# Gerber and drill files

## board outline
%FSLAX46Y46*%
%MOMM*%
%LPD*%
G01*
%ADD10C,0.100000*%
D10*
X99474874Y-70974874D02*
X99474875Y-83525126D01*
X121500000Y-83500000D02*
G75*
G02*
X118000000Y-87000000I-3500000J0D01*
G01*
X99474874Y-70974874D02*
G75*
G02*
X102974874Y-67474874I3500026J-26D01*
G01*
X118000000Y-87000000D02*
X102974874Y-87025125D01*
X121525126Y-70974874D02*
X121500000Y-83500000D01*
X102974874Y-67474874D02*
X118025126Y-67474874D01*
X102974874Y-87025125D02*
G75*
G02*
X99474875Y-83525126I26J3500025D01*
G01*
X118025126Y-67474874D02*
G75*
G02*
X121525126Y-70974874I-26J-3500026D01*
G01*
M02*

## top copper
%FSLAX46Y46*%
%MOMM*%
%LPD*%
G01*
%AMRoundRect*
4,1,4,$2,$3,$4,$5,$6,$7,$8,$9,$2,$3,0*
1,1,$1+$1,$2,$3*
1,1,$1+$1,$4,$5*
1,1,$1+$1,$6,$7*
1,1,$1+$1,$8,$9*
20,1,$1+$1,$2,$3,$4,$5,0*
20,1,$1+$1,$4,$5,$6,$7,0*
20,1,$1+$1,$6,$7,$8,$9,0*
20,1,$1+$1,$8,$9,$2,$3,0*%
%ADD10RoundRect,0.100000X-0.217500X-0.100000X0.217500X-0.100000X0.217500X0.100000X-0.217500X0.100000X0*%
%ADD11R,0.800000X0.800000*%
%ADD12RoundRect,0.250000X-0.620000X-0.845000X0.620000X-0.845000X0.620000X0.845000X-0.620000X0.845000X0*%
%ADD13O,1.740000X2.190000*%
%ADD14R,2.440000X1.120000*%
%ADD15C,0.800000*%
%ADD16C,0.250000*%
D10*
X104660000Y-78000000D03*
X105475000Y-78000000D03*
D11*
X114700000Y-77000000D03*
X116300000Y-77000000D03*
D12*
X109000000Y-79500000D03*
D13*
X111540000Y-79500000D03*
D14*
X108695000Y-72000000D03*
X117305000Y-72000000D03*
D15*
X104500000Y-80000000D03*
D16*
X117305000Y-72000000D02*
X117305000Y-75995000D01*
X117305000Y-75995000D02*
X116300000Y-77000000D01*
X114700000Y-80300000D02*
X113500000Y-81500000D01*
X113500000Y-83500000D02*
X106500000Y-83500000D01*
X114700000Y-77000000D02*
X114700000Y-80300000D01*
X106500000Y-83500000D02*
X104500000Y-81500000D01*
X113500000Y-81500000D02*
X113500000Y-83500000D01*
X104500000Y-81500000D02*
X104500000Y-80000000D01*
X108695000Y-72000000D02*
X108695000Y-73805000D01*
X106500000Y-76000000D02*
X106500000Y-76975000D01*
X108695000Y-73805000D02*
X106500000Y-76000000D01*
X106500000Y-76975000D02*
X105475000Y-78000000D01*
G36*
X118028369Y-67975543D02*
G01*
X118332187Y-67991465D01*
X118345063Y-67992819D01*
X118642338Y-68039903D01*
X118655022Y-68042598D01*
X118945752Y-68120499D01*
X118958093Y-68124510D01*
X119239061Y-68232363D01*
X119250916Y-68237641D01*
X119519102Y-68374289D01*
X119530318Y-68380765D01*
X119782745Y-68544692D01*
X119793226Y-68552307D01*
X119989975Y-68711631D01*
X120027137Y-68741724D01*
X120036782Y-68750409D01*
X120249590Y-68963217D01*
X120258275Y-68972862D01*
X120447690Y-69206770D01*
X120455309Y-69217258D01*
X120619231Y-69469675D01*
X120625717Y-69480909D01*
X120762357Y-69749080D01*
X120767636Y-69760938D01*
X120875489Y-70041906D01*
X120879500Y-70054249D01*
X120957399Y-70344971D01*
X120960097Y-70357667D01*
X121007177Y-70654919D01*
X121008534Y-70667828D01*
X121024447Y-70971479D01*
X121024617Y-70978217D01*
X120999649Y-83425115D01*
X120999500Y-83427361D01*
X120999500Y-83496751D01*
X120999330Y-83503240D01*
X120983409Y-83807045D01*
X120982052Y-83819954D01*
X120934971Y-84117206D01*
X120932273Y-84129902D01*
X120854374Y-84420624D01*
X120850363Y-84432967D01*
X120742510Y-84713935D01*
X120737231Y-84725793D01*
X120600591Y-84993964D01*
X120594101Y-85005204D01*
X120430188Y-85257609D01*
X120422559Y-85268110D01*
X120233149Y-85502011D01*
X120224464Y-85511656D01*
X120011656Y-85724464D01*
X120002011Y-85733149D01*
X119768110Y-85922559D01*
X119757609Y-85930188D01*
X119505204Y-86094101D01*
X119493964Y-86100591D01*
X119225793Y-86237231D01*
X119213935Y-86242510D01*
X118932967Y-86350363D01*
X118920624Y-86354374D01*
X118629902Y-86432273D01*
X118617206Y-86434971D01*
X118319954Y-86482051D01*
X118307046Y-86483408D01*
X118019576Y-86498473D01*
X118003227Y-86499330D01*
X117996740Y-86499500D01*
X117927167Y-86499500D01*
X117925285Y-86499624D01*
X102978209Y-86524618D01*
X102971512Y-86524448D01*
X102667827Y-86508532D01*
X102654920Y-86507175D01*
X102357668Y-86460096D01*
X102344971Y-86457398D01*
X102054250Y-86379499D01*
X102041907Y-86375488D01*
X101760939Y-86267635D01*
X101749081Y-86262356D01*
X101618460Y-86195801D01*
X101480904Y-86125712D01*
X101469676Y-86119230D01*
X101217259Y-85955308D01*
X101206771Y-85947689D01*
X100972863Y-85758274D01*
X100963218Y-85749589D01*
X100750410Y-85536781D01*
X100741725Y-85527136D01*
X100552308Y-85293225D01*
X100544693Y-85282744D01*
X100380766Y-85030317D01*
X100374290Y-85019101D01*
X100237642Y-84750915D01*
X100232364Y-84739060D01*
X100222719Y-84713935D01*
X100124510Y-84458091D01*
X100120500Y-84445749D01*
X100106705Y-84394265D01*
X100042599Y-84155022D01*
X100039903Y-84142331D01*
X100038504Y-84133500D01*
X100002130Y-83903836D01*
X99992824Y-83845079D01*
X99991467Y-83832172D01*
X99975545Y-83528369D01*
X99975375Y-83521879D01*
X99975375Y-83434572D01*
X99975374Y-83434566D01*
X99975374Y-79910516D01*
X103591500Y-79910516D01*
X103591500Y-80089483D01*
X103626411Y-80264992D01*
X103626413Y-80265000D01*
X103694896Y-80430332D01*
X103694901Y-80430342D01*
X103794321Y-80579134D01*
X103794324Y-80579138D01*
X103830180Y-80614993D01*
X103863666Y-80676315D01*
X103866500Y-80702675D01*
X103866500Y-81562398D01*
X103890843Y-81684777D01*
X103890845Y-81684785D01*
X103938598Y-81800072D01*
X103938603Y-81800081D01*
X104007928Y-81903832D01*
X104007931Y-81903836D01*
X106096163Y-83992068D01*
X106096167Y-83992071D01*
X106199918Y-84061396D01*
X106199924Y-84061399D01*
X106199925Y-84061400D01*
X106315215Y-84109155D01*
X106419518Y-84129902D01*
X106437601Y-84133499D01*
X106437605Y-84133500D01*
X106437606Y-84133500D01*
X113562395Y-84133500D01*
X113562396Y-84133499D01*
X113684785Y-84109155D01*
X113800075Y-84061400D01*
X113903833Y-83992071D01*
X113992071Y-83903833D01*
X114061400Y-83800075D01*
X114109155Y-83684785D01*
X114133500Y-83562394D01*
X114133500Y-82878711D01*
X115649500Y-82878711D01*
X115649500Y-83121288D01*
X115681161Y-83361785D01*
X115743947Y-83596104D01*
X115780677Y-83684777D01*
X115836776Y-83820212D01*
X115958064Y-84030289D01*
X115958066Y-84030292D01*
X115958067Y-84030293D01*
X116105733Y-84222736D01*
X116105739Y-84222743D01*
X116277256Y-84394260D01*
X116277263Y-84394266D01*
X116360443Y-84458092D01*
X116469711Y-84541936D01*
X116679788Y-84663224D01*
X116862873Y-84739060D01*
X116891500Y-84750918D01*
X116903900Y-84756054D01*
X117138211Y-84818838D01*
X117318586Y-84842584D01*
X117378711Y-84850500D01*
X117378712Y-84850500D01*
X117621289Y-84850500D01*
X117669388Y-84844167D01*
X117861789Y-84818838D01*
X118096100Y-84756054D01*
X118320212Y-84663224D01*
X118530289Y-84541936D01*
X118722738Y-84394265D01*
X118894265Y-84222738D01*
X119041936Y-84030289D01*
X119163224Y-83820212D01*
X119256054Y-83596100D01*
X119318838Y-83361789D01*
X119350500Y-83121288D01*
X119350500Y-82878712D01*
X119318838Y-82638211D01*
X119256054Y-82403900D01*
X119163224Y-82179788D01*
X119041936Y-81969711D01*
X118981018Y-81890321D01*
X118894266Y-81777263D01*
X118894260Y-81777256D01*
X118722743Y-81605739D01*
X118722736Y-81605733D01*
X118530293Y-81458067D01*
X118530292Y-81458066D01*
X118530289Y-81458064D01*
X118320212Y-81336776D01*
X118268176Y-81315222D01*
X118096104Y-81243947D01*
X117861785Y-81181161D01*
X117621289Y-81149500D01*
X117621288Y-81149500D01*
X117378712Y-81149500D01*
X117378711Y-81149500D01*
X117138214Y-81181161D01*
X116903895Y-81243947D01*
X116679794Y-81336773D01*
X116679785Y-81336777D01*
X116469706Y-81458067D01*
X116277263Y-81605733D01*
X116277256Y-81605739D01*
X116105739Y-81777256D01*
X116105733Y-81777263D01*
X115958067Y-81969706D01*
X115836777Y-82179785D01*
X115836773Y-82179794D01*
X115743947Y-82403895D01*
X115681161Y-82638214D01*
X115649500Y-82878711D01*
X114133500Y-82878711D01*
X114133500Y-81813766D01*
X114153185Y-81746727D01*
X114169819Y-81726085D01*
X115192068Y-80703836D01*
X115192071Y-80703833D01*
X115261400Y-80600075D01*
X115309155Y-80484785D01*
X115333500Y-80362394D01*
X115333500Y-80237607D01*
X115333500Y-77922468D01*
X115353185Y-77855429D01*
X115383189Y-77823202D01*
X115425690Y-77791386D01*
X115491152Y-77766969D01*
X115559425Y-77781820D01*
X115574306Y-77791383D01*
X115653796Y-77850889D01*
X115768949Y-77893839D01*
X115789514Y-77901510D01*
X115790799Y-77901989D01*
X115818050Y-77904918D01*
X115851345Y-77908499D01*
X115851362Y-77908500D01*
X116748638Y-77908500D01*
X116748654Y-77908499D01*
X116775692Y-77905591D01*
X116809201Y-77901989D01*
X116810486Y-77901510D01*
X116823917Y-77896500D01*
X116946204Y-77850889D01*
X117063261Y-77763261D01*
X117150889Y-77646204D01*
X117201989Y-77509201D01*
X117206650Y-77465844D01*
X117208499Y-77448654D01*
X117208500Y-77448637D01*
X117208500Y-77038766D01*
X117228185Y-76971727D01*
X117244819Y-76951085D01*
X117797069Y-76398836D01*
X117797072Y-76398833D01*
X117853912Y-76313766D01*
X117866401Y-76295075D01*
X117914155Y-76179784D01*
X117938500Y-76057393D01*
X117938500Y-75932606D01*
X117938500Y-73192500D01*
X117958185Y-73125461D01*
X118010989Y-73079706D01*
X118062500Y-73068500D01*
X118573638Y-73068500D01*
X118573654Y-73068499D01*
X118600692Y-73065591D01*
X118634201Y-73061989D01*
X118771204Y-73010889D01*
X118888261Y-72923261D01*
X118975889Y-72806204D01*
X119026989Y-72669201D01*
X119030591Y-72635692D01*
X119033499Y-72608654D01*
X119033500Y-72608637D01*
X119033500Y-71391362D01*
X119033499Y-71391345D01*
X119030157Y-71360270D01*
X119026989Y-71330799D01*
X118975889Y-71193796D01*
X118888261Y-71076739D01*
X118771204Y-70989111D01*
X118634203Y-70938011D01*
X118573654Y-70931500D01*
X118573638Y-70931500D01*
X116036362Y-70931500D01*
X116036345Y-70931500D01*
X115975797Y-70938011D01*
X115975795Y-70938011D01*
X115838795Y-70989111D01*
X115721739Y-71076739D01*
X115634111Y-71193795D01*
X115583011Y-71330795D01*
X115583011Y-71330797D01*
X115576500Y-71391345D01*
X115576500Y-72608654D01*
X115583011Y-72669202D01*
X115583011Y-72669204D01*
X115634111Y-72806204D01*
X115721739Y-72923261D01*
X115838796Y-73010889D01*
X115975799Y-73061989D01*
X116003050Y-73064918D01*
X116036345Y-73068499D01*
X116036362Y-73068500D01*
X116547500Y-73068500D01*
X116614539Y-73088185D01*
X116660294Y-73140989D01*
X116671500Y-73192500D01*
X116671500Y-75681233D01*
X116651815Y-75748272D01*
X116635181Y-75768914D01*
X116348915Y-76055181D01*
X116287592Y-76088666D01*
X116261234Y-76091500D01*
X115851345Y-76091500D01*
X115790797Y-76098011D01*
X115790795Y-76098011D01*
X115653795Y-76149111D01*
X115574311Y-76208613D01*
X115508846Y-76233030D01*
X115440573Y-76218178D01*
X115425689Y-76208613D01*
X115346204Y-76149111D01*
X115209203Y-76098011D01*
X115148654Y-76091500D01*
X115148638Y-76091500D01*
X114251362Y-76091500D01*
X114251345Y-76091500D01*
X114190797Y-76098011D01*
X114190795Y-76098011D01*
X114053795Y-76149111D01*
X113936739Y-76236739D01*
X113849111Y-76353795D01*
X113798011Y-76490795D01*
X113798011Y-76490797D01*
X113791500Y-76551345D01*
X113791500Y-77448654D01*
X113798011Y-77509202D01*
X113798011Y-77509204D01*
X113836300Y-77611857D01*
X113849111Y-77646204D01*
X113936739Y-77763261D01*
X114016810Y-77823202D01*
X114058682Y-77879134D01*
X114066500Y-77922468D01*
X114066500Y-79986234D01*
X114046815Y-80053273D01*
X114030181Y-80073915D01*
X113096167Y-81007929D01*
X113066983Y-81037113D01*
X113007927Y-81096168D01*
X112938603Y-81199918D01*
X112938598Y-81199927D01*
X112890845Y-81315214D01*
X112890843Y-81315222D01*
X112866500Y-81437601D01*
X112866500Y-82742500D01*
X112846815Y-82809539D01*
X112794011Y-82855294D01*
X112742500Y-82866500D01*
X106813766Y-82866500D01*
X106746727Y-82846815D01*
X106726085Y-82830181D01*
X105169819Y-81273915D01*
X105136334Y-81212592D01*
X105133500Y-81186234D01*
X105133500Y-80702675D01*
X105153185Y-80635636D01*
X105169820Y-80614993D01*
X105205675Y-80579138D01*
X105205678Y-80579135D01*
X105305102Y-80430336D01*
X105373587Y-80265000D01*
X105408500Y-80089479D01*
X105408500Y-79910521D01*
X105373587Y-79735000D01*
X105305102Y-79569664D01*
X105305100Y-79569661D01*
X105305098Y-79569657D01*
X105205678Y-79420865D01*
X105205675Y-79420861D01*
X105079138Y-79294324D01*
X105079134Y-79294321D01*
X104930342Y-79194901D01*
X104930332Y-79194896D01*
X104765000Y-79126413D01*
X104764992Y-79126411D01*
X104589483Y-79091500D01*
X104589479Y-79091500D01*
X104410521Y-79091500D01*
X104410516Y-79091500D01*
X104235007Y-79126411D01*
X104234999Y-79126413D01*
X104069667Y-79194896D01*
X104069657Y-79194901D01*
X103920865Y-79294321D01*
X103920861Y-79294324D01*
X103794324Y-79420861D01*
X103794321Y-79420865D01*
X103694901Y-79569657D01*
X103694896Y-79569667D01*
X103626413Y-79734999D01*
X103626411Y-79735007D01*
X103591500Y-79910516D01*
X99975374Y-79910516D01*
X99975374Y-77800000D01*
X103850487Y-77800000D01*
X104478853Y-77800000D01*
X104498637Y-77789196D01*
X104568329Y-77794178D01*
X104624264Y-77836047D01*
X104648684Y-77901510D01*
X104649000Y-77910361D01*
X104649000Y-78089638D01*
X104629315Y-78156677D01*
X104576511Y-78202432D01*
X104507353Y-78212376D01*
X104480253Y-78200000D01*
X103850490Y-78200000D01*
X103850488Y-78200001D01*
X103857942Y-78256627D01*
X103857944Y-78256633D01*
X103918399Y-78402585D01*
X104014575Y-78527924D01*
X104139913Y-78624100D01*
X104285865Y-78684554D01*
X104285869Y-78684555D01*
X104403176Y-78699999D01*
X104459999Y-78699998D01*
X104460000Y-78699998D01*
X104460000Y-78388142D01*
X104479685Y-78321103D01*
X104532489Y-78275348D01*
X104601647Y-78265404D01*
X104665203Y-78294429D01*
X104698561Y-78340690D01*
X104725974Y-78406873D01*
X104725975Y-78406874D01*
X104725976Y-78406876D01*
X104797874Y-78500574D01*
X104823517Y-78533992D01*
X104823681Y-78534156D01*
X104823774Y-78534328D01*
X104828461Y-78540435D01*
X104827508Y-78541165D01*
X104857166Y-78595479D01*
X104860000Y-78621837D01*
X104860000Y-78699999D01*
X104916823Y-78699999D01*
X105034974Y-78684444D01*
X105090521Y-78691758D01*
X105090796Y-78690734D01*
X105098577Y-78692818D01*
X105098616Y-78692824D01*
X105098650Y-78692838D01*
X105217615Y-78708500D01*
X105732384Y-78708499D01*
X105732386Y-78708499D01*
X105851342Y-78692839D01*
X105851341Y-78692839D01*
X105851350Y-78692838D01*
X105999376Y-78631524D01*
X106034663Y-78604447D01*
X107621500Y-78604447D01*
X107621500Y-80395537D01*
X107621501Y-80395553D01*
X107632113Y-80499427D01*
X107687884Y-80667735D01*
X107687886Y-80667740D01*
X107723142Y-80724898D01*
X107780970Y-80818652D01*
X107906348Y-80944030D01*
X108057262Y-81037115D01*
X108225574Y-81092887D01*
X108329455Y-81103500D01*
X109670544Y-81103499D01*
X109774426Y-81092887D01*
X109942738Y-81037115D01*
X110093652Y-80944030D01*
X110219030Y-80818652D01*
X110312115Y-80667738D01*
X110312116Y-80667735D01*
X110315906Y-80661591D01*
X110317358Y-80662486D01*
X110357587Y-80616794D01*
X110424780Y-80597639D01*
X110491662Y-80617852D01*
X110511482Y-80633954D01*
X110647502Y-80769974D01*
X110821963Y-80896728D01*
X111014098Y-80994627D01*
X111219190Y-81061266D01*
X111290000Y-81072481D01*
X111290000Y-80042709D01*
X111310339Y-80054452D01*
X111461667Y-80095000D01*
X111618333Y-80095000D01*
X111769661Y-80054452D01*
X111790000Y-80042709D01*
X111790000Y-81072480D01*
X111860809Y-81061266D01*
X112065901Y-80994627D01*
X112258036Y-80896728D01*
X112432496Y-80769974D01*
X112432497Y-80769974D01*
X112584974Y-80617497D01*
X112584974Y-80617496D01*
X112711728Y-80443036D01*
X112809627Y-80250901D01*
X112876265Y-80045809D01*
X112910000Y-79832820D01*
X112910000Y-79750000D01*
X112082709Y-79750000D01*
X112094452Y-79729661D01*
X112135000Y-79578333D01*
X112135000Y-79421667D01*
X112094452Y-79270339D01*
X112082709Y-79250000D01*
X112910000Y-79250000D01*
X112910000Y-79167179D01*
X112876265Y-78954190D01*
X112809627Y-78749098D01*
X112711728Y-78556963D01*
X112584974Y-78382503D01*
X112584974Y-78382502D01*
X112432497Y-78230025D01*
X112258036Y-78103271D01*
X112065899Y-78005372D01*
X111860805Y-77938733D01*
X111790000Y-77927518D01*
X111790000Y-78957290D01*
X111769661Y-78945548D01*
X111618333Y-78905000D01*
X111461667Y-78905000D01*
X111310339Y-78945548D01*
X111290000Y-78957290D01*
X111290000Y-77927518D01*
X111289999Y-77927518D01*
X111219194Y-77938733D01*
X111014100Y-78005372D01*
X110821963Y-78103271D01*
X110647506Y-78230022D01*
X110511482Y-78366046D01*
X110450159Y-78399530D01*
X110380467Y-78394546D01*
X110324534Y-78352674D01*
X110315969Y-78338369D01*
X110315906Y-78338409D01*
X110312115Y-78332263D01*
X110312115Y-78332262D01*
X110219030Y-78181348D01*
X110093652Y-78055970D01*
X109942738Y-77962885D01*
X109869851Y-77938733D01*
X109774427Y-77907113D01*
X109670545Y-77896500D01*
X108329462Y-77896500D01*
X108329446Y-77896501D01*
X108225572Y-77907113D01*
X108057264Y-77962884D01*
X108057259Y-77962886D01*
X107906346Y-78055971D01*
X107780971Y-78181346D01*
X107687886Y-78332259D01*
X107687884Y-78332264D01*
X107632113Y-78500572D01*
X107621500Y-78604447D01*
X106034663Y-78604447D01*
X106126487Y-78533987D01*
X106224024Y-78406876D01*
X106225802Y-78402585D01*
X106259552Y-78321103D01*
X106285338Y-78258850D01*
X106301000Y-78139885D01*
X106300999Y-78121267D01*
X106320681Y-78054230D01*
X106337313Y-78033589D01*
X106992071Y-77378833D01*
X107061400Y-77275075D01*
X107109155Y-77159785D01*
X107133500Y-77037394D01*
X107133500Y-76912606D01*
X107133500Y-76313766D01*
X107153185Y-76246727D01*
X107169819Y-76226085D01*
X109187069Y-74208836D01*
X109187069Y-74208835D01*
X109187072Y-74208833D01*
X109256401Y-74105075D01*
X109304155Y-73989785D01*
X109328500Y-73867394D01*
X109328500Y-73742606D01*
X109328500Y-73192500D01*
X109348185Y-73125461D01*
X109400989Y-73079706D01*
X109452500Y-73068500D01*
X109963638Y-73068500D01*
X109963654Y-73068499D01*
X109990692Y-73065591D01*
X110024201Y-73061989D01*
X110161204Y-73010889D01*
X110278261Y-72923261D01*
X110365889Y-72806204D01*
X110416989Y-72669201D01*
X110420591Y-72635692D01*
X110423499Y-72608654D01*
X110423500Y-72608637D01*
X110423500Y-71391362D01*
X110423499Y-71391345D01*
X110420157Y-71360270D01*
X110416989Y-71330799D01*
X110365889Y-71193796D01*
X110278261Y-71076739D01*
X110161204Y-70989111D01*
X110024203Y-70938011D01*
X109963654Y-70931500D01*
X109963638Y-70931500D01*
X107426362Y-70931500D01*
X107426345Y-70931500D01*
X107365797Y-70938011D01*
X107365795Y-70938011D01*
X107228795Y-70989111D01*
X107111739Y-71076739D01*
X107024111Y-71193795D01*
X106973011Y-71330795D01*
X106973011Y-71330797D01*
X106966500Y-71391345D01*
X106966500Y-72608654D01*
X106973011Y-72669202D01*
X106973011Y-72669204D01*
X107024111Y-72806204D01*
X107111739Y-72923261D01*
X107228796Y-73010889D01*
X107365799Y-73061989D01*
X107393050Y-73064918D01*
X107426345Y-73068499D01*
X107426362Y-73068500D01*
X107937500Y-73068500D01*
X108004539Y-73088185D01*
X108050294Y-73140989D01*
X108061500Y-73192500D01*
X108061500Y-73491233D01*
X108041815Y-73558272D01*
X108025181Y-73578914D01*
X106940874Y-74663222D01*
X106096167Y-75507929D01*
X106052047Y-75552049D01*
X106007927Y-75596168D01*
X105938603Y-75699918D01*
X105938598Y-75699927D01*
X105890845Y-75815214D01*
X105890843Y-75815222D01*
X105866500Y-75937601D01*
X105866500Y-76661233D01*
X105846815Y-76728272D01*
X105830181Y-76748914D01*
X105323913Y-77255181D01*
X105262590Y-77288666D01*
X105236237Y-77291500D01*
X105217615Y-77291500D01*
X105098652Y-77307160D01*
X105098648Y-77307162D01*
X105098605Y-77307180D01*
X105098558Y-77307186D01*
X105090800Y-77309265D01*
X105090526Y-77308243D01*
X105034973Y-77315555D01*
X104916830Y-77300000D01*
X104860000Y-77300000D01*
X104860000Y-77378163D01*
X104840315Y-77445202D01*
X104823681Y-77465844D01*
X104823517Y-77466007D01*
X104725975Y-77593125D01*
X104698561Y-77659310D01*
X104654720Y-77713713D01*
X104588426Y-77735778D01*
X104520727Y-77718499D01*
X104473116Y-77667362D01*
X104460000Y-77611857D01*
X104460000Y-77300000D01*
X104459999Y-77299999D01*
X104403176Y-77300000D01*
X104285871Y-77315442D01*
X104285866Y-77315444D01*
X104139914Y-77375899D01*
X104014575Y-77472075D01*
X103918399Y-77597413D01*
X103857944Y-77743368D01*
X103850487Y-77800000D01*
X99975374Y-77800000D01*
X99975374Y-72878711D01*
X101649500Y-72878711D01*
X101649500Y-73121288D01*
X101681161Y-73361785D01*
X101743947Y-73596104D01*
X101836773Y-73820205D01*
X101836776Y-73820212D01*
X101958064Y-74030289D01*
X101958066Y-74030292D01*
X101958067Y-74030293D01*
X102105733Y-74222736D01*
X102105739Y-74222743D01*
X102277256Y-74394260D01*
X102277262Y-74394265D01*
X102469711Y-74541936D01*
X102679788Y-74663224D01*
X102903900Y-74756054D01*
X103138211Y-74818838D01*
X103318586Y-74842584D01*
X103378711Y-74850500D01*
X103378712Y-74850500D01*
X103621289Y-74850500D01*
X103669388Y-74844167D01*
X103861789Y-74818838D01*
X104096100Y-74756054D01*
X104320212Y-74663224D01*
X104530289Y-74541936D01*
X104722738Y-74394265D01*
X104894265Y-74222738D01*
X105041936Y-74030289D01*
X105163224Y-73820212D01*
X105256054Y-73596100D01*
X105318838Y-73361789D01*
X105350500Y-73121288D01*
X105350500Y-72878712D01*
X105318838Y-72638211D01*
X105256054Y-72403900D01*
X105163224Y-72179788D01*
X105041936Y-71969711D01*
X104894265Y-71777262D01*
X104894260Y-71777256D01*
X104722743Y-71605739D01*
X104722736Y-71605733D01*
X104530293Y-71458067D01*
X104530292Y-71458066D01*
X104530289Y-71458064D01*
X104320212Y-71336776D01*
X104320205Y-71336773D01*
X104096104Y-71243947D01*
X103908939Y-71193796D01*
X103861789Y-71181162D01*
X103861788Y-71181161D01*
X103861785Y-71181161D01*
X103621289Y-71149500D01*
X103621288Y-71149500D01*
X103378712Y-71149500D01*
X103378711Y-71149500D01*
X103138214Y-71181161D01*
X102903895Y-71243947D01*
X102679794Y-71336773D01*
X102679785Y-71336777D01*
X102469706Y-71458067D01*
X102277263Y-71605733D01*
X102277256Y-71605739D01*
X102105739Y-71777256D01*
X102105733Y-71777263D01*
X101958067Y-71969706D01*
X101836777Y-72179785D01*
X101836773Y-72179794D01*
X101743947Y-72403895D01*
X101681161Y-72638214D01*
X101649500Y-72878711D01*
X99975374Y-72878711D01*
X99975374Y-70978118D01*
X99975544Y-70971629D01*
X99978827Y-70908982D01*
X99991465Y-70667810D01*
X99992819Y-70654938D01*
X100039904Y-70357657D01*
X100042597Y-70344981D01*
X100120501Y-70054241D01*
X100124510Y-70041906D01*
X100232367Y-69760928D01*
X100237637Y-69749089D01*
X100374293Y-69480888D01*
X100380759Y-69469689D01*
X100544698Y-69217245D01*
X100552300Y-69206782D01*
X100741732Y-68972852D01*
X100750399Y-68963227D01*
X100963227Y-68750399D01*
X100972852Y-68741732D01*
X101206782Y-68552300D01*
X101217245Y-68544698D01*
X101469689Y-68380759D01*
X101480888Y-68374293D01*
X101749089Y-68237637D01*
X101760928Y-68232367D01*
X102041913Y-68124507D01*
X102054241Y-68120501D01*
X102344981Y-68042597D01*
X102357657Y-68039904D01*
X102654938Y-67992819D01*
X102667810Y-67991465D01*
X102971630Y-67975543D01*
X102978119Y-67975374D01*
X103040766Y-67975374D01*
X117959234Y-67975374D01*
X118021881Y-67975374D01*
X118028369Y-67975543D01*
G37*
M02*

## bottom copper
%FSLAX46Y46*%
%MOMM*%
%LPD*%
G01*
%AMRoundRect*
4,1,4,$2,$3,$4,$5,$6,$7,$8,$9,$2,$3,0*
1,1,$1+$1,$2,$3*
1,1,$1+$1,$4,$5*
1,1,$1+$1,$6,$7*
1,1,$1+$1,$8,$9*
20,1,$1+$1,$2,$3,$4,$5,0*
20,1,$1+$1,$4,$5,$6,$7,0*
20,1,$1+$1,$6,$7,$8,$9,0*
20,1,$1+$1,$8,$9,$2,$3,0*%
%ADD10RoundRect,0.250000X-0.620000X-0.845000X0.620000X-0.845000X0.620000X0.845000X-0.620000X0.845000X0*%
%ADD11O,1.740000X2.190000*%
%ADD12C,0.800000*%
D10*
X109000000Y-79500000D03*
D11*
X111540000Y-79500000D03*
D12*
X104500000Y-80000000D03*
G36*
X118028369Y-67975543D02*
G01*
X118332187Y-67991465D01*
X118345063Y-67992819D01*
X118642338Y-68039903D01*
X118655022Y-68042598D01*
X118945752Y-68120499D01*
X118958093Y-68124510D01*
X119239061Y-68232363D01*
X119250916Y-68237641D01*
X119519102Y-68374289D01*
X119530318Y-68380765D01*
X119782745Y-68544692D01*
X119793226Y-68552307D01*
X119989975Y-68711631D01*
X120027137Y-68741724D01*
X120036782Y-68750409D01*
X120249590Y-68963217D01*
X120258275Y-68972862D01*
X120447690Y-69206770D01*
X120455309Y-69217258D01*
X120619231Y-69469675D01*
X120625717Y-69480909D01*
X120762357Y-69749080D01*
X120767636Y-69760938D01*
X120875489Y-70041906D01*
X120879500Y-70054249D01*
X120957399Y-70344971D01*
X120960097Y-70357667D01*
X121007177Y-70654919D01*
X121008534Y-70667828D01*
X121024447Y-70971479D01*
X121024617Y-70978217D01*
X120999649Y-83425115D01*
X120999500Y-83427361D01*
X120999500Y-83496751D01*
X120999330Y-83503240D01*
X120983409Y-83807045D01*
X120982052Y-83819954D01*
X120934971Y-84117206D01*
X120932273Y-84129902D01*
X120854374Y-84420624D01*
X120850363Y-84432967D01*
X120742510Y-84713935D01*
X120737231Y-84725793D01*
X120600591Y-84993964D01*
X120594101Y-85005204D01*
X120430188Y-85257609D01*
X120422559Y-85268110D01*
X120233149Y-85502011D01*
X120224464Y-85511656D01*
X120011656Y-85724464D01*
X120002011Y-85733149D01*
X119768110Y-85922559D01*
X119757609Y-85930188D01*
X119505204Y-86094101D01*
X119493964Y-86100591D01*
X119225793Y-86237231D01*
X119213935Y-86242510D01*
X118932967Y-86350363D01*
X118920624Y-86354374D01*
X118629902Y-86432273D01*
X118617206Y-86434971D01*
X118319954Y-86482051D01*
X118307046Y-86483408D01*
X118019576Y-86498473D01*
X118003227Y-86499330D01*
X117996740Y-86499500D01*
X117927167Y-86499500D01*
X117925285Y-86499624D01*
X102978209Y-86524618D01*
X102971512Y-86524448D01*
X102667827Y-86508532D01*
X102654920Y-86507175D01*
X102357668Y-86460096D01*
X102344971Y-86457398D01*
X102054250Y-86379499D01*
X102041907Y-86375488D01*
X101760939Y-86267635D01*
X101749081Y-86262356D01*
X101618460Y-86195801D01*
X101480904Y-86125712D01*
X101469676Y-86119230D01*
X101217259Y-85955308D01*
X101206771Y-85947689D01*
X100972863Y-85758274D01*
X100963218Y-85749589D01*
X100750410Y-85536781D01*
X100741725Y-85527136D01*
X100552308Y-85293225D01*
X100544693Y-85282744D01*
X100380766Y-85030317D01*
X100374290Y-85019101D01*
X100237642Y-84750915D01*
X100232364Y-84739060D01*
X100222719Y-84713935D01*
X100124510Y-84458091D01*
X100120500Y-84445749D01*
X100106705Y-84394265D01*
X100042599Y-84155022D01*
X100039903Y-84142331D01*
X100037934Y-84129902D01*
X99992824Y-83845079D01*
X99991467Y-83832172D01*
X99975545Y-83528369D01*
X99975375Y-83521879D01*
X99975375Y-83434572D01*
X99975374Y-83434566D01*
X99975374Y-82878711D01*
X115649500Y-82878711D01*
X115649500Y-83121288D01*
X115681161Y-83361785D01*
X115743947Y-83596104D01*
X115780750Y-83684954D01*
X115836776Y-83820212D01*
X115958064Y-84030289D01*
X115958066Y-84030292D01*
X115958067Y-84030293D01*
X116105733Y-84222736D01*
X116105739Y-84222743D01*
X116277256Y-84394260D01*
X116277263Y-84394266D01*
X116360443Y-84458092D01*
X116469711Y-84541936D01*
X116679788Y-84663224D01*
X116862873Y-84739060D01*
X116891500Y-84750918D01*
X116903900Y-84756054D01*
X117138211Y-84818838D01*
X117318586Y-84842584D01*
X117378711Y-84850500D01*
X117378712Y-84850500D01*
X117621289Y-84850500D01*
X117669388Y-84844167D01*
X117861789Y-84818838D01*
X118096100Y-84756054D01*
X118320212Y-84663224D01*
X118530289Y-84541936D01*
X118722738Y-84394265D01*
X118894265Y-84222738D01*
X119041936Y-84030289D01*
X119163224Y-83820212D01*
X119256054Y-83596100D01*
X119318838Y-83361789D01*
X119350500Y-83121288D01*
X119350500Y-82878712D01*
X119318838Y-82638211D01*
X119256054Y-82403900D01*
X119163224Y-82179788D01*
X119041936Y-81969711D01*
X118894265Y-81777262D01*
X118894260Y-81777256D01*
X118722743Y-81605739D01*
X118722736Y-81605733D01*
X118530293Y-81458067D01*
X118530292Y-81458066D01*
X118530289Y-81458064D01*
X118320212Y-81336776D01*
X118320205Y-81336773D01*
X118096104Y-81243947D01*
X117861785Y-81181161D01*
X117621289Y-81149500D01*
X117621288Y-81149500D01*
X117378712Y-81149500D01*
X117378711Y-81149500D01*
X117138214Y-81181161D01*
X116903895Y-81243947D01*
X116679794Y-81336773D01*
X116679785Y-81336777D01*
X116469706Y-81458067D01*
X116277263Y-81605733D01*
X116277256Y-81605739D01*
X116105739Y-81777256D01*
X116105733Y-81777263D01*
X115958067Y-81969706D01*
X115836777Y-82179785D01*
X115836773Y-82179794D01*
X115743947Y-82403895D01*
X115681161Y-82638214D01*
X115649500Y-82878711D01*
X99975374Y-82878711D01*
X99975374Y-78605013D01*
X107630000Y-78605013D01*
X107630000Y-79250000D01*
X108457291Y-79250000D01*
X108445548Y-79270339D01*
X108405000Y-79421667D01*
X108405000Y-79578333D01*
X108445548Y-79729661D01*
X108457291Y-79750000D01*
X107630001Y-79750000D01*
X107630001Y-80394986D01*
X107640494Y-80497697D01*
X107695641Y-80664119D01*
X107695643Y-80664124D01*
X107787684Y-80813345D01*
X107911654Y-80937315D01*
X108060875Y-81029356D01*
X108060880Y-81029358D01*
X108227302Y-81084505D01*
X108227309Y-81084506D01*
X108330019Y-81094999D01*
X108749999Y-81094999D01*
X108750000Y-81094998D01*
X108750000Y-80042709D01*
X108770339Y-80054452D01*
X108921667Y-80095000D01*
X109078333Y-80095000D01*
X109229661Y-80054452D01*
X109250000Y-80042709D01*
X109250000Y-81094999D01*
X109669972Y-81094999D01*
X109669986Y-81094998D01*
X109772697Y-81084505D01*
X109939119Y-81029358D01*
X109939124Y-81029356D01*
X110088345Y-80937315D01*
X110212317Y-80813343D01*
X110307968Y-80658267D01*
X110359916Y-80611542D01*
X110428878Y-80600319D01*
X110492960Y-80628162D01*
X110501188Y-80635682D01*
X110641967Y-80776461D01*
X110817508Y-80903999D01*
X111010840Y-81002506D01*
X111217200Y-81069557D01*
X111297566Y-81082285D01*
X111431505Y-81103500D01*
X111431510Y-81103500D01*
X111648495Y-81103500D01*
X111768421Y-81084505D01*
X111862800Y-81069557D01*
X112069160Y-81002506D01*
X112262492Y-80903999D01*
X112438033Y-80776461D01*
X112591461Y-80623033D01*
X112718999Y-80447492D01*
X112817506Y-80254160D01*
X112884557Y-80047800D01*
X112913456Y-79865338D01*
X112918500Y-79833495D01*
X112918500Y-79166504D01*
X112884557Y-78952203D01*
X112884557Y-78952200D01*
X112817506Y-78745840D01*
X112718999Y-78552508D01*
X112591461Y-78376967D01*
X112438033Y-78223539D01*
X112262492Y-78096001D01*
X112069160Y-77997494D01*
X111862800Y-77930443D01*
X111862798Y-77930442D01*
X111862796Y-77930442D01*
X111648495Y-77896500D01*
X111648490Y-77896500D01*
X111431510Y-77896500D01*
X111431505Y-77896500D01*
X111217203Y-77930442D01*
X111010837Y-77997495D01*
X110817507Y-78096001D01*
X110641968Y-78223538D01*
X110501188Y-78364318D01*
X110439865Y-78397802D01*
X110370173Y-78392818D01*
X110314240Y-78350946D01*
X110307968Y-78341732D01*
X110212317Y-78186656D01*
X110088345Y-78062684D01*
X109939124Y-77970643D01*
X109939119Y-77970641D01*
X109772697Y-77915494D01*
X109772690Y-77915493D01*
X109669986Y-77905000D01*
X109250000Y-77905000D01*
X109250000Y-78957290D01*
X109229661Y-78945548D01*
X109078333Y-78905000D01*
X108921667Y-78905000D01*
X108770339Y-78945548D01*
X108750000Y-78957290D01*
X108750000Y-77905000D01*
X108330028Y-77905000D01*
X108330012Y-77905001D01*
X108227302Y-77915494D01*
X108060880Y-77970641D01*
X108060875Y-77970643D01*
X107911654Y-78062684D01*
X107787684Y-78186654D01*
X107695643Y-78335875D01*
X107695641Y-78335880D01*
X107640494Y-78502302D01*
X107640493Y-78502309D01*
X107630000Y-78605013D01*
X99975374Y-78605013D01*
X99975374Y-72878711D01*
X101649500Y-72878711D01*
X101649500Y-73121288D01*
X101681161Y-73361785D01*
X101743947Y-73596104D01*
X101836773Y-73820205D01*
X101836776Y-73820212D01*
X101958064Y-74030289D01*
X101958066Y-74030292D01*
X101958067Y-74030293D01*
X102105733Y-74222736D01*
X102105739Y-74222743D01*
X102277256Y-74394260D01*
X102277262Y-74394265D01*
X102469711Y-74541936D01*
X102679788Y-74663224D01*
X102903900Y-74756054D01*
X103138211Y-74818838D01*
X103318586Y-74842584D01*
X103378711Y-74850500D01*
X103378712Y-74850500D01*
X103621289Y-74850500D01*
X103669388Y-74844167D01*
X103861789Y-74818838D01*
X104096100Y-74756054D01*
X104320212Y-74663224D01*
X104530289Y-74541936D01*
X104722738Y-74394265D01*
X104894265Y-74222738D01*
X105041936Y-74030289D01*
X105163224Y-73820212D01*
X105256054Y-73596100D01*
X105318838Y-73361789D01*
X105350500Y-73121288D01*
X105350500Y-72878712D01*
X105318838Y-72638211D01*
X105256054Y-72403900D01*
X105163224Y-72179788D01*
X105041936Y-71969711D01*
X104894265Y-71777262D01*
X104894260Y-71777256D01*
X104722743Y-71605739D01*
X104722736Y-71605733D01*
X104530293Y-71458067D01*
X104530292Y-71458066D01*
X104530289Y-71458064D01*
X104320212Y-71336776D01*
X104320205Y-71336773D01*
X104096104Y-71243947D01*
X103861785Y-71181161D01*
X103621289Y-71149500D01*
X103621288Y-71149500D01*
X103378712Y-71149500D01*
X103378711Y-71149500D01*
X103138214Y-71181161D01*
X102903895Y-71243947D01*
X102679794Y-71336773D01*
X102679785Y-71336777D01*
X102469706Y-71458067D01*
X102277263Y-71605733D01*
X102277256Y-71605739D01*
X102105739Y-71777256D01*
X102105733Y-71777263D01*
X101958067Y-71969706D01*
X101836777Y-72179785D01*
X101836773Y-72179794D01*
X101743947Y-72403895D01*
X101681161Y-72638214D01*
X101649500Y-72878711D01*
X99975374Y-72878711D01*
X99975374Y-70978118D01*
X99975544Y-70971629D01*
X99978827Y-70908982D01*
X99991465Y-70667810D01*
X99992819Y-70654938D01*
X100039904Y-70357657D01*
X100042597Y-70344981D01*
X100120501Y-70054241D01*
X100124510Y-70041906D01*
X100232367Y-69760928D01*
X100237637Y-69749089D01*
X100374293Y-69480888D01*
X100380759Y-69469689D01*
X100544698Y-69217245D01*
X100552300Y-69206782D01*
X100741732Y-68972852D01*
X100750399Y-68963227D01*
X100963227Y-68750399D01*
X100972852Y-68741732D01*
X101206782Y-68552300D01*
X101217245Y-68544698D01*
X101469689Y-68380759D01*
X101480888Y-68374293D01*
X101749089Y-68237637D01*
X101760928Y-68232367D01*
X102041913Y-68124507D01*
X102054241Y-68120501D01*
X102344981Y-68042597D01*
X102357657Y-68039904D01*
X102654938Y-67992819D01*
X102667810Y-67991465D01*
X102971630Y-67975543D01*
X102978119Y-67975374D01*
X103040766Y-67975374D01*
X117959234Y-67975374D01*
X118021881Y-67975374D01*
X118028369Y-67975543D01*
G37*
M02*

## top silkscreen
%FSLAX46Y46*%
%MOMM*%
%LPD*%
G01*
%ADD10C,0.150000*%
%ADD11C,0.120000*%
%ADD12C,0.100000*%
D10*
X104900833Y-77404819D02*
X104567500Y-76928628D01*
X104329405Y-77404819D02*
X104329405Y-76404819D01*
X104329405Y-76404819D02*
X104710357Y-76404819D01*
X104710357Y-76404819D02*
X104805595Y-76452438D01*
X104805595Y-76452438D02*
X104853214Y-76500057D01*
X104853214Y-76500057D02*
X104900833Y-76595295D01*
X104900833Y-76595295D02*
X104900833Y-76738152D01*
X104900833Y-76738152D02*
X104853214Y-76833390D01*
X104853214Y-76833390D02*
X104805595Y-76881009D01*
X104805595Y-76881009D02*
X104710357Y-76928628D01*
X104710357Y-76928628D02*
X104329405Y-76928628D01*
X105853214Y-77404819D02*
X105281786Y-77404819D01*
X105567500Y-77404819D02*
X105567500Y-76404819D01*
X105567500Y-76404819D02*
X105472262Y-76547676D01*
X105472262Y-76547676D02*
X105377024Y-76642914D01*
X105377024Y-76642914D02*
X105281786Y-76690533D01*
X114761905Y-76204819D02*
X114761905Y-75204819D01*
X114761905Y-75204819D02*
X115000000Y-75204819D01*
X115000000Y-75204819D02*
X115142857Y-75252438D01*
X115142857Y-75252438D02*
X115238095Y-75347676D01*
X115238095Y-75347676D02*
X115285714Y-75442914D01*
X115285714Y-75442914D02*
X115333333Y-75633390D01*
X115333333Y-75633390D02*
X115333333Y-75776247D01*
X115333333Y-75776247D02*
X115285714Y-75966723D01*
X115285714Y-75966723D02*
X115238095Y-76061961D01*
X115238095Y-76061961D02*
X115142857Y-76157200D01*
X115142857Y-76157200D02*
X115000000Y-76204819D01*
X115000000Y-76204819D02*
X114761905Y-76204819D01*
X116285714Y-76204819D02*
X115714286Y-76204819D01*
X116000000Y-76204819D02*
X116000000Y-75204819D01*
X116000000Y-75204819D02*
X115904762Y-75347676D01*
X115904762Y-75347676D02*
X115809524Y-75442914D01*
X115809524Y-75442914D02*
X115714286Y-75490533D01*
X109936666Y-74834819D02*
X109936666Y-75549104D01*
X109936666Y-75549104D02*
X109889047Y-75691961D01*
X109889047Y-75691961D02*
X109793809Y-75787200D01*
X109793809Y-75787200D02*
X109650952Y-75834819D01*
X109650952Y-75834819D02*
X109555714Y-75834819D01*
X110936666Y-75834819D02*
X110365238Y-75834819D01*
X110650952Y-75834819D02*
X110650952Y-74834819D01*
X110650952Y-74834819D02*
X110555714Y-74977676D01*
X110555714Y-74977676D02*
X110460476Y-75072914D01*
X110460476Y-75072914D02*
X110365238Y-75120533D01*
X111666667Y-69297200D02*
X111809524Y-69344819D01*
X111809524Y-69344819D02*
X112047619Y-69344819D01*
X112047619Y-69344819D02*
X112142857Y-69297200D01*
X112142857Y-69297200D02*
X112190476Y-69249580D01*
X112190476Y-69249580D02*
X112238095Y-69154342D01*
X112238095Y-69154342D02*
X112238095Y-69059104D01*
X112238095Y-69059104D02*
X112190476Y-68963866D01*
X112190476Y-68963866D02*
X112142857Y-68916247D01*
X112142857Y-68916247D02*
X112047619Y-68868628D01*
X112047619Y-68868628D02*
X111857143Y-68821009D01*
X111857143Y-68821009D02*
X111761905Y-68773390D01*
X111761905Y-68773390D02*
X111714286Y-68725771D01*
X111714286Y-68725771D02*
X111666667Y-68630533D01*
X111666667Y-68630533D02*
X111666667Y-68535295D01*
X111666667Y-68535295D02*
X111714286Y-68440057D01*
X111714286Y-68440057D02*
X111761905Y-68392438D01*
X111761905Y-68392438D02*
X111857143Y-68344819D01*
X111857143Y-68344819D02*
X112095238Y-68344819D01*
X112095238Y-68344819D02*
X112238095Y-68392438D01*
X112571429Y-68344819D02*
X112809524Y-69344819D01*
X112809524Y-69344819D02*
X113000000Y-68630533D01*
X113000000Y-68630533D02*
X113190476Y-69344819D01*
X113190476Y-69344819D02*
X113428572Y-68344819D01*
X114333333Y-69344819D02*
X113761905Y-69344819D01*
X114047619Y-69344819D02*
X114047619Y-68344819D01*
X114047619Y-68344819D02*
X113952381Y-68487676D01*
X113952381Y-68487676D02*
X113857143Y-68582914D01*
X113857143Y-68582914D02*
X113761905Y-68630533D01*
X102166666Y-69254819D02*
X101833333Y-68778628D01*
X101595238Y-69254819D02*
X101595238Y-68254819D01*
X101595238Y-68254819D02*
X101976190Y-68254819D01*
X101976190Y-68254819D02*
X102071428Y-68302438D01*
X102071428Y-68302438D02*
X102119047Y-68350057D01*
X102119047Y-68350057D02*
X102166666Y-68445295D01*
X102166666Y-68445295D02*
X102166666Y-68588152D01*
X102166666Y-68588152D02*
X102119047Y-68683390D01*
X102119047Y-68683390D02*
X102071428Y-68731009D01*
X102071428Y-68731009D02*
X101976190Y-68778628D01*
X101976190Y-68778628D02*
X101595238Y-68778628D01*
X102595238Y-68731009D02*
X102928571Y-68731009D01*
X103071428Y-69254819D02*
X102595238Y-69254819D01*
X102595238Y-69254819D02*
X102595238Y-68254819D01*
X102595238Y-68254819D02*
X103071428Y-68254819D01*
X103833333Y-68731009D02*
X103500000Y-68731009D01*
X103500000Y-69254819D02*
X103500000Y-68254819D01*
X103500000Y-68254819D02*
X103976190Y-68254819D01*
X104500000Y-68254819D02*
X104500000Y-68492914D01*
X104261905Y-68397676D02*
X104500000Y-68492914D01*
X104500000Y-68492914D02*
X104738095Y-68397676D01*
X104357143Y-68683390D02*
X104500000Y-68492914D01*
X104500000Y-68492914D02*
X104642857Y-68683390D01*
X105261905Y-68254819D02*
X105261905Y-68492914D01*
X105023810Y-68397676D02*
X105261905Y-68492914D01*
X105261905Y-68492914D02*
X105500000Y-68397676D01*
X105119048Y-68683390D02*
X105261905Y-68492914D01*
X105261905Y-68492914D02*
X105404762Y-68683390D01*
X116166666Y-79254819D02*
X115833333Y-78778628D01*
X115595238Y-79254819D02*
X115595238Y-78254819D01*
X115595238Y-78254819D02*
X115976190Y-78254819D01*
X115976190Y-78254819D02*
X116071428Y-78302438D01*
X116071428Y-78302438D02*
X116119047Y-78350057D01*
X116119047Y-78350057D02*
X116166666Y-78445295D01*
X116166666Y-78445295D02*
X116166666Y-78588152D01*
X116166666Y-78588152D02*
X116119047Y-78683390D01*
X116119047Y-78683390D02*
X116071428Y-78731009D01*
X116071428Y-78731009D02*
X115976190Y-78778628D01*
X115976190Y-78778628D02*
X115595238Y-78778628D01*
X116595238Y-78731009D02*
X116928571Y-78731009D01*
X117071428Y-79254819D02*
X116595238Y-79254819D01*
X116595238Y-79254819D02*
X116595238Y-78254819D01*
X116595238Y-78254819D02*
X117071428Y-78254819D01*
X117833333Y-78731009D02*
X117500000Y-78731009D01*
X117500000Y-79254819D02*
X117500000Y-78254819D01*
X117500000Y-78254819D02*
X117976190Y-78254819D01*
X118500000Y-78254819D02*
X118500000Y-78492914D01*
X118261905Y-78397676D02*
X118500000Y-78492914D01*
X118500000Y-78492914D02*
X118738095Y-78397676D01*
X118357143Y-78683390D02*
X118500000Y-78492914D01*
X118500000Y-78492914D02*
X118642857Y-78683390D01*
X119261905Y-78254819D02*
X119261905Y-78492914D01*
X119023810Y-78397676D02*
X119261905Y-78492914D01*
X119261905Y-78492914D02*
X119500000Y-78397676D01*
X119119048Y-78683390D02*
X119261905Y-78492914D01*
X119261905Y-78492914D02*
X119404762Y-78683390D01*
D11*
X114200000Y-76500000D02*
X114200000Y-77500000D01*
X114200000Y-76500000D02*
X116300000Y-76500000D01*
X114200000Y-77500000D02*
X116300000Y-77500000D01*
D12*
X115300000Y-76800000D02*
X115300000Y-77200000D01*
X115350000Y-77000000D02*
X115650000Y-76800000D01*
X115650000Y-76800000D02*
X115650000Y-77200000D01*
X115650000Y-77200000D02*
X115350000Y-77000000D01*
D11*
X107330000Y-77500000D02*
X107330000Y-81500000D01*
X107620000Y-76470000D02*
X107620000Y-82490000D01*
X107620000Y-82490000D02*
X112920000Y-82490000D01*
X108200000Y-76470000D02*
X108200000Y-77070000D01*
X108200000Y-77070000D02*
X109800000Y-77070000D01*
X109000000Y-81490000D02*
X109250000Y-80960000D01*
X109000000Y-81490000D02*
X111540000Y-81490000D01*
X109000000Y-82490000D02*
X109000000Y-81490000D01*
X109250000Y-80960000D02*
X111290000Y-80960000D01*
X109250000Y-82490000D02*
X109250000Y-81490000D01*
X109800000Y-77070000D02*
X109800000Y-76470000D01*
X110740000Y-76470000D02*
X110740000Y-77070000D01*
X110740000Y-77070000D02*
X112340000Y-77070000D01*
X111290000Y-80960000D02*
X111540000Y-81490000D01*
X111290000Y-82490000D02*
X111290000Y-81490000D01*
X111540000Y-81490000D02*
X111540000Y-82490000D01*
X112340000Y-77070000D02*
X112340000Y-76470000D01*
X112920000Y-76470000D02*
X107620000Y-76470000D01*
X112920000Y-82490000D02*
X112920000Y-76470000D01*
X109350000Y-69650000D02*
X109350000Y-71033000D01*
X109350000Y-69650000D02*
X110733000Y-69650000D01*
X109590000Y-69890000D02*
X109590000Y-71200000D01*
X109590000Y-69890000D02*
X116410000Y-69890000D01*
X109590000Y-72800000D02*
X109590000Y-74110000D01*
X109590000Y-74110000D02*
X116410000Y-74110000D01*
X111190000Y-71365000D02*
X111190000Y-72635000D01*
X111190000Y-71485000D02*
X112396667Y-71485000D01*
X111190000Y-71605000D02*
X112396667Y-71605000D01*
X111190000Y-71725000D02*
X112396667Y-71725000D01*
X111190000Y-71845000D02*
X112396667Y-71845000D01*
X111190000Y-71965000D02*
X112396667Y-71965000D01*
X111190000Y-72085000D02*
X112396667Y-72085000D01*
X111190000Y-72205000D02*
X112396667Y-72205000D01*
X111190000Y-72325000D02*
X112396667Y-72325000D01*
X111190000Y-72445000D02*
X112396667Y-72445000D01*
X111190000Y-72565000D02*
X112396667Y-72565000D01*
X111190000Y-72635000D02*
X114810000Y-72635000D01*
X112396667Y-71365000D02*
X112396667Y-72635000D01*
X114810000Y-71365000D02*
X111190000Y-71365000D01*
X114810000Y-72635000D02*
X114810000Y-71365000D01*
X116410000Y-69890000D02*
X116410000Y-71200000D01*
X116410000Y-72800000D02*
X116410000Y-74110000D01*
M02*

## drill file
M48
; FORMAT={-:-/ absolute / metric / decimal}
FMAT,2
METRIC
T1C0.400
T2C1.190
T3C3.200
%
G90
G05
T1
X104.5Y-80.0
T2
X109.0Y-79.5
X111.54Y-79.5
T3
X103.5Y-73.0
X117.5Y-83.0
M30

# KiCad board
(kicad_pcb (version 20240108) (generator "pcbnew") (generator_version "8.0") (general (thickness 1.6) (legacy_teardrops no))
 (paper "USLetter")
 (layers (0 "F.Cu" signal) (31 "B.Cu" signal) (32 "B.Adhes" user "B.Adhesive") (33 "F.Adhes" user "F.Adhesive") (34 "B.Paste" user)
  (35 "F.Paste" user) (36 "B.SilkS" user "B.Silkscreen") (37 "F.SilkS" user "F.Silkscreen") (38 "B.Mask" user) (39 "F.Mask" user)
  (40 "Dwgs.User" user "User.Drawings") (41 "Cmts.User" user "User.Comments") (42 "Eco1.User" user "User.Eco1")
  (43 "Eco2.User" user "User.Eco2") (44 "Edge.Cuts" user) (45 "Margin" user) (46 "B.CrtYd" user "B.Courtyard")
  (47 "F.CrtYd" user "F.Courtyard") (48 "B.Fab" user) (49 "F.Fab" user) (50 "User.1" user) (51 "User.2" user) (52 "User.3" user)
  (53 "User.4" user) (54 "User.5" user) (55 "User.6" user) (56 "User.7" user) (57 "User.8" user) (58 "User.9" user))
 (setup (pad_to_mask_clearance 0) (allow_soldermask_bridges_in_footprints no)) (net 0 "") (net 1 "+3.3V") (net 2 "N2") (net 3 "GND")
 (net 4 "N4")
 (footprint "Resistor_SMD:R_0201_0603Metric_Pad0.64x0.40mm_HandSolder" (layer "F.Cu") (at 105.0675 78)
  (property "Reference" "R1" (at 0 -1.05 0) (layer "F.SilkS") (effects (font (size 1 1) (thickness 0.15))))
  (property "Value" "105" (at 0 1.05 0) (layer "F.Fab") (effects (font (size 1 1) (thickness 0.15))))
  (pad "" smd roundrect (at -0.4325 0) (size 0.458 0.36) (layers "F.Paste") (roundrect_rratio 0.25))
  (pad "" smd roundrect (at 0.4325 0) (size 0.458 0.36) (layers "F.Paste") (roundrect_rratio 0.25))
  (pad "1" smd roundrect (at -0.4075 0) (size 0.635 0.4) (layers "F.Cu" "F.Mask") (roundrect_rratio 0.25) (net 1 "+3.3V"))
  (pad "2" smd roundrect (at 0.4075 0) (size 0.635 0.4) (layers "F.Cu" "F.Mask") (roundrect_rratio 0.25) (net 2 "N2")))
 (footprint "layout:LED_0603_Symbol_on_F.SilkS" (layer "F.Cu") (at 115.5 77)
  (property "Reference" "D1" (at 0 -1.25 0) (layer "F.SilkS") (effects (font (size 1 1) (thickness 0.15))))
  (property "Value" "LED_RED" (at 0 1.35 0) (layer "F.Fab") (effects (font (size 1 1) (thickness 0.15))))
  (fp_line (start -1.3 -0.5) (end -1.3 0.5) (stroke (width 0.12) (type solid)) (layer "F.SilkS"))
  (fp_line (start -1.3 -0.5) (end 0.8 -0.5) (stroke (width 0.12) (type solid)) (layer "F.SilkS"))
  (fp_line (start -1.3 0.5) (end 0.8 0.5) (stroke (width 0.12) (type solid)) (layer "F.SilkS"))
  (fp_line (start -0.2 -0.2) (end -0.2 0.2) (stroke (width 0.1) (type solid)) (layer "F.SilkS"))
  (fp_line (start -0.15 0) (end 0.15 -0.2) (stroke (width 0.1) (type solid)) (layer "F.SilkS"))
  (fp_line (start 0.15 -0.2) (end 0.15 0.2) (stroke (width 0.1) (type solid)) (layer "F.SilkS"))
  (fp_line (start 0.15 0.2) (end -0.15 0) (stroke (width 0.1) (type solid)) (layer "F.SilkS"))
  (pad "1" smd rect (at -0.8 0 180) (size 0.8 0.8) (layers "F.Cu" "F.Paste" "F.Mask") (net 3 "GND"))
  (pad "2" smd rect (at 0.8 0 180) (size 0.8 0.8) (layers "F.Cu" "F.Paste" "F.Mask") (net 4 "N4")))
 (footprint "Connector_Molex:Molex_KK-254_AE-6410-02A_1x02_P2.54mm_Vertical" (layer "F.Cu") (at 109 79.5)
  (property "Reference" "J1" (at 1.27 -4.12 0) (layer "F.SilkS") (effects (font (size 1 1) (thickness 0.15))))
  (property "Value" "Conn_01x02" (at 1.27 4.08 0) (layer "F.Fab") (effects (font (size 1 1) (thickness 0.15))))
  (fp_line (start -1.67 -2) (end -1.67 2) (stroke (width 0.12) (type solid)) (layer "F.SilkS"))
  (fp_line (start -1.38 -3.03) (end -1.38 2.99) (stroke (width 0.12) (type solid)) (layer "F.SilkS"))
  (fp_line (start -1.38 2.99) (end 3.92 2.99) (stroke (width 0.12) (type solid)) (layer "F.SilkS"))
  (fp_line (start -0.8 -3.03) (end -0.8 -2.43) (stroke (width 0.12) (type solid)) (layer "F.SilkS"))
  (fp_line (start -0.8 -2.43) (end 0.8 -2.43) (stroke (width 0.12) (type solid)) (layer "F.SilkS"))
  (fp_line (start 0 1.99) (end 0.25 1.46) (stroke (width 0.12) (type solid)) (layer "F.SilkS"))
  (fp_line (start 0 1.99) (end 2.54 1.99) (stroke (width 0.12) (type solid)) (layer "F.SilkS"))
  (fp_line (start 0 2.99) (end 0 1.99) (stroke (width 0.12) (type solid)) (layer "F.SilkS"))
  (fp_line (start 0.25 1.46) (end 2.29 1.46) (stroke (width 0.12) (type solid)) (layer "F.SilkS"))
  (fp_line (start 0.25 2.99) (end 0.25 1.99) (stroke (width 0.12) (type solid)) (layer "F.SilkS"))
  (fp_line (start 0.8 -2.43) (end 0.8 -3.03) (stroke (width 0.12) (type solid)) (layer "F.SilkS"))
  (fp_line (start 1.74 -3.03) (end 1.74 -2.43) (stroke (width 0.12) (type solid)) (layer "F.SilkS"))
  (fp_line (start 1.74 -2.43) (end 3.34 -2.43) (stroke (width 0.12) (type solid)) (layer "F.SilkS"))
  (fp_line (start 2.29 1.46) (end 2.54 1.99) (stroke (width 0.12) (type solid)) (layer "F.SilkS"))
  (fp_line (start 2.29 2.99) (end 2.29 1.99) (stroke (width 0.12) (type solid)) (layer "F.SilkS"))
  (fp_line (start 2.54 1.99) (end 2.54 2.99) (stroke (width 0.12) (type solid)) (layer "F.SilkS"))
  (fp_line (start 3.34 -2.43) (end 3.34 -3.03) (stroke (width 0.12) (type solid)) (layer "F.SilkS"))
  (fp_line (start 3.92 -3.03) (end -1.38 -3.03) (stroke (width 0.12) (type solid)) (layer "F.SilkS"))
  (fp_line (start 3.92 2.99) (end 3.92 -3.03) (stroke (width 0.12) (type solid)) (layer "F.SilkS"))
  (pad "1" thru_hole roundrect (at 0 0) (size 1.74 2.19) (drill 1.19) (layers "*.Cu" "*.Mask") (remove_unused_layers no)
   (roundrect_rratio 0.143678) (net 3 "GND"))
  (pad "2" thru_hole oval (at 2.54 0) (size 1.74 2.19) (drill 1.19) (layers "*.Cu" "*.Mask") (remove_unused_layers no) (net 1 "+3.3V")))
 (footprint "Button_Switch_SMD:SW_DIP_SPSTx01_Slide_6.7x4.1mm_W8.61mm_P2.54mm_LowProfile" (layer "F.Cu") (at 113 72)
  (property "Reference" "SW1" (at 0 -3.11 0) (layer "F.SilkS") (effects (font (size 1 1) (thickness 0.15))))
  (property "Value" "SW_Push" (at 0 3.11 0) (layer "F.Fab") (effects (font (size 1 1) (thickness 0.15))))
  (fp_line (start -3.65 -2.35) (end -3.65 -0.967) (stroke (width 0.12) (type solid)) (layer "F.SilkS"))
  (fp_line (start -3.65 -2.35) (end -2.267 -2.35) (stroke (width 0.12) (type solid)) (layer "F.SilkS"))
  (fp_line (start -3.41 -2.11) (end -3.41 -0.8) (stroke (width 0.12) (type solid)) (layer "F.SilkS"))
  (fp_line (start -3.41 -2.11) (end 3.41 -2.11) (stroke (width 0.12) (type solid)) (layer "F.SilkS"))
  (fp_line (start -3.41 0.8) (end -3.41 2.11) (stroke (width 0.12) (type solid)) (layer "F.SilkS"))
  (fp_line (start -3.41 2.11) (end 3.41 2.11) (stroke (width 0.12) (type solid)) (layer "F.SilkS"))
  (fp_line (start -1.81 -0.635) (end -1.81 0.635) (stroke (width 0.12) (type solid)) (layer "F.SilkS"))
  (fp_line (start -1.81 -0.515) (end -0.603333 -0.515) (stroke (width 0.12) (type solid)) (layer "F.SilkS"))
  (fp_line (start -1.81 -0.395) (end -0.603333 -0.395) (stroke (width 0.12) (type solid)) (layer "F.SilkS"))
  (fp_line (start -1.81 -0.275) (end -0.603333 -0.275) (stroke (width 0.12) (type solid)) (layer "F.SilkS"))
  (fp_line (start -1.81 -0.155) (end -0.603333 -0.155) (stroke (width 0.12) (type solid)) (layer "F.SilkS"))
  (fp_line (start -1.81 -0.035) (end -0.603333 -0.035) (stroke (width 0.12) (type solid)) (layer "F.SilkS"))
  (fp_line (start -1.81 0.085) (end -0.603333 0.085) (stroke (width 0.12) (type solid)) (layer "F.SilkS"))
  (fp_line (start -1.81 0.205) (end -0.603333 0.205) (stroke (width 0.12) (type solid)) (layer "F.SilkS"))
  (fp_line (start -1.81 0.325) (end -0.603333 0.325) (stroke (width 0.12) (type solid)) (layer "F.SilkS"))
  (fp_line (start -1.81 0.445) (end -0.603333 0.445) (stroke (width 0.12) (type solid)) (layer "F.SilkS"))
  (fp_line (start -1.81 0.565) (end -0.603333 0.565) (stroke (width 0.12) (type solid)) (layer "F.SilkS"))
  (fp_line (start -1.81 0.635) (end 1.81 0.635) (stroke (width 0.12) (type solid)) (layer "F.SilkS"))
  (fp_line (start -0.603333 -0.635) (end -0.603333 0.635) (stroke (width 0.12) (type solid)) (layer "F.SilkS"))
  (fp_line (start 1.81 -0.635) (end -1.81 -0.635) (stroke (width 0.12) (type solid)) (layer "F.SilkS"))
  (fp_line (start 1.81 0.635) (end 1.81 -0.635) (stroke (width 0.12) (type solid)) (layer "F.SilkS"))
  (fp_line (start 3.41 -2.11) (end 3.41 -0.8) (stroke (width 0.12) (type solid)) (layer "F.SilkS"))
  (fp_line (start 3.41 0.8) (end 3.41 2.11) (stroke (width 0.12) (type solid)) (layer "F.SilkS"))
  (pad "1" smd rect (at -4.305 0) (size 2.44 1.12) (layers "F.Cu" "F.Paste" "F.Mask") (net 2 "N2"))
  (pad "2" smd rect (at 4.305 0) (size 2.44 1.12) (layers "F.Cu" "F.Paste" "F.Mask") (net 4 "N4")))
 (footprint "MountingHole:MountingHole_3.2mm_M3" (layer "F.Cu") (at 103.5 73)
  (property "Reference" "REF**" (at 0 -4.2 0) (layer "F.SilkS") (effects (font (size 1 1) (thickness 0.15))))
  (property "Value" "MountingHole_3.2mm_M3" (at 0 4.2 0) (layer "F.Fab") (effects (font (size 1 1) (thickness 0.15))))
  (pad "" np_thru_hole circle (at 0 0) (size 3.2 3.2) (drill 3.2) (layers "*.Cu" "*.Mask")))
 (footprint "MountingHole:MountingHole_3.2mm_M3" (layer "F.Cu") (at 117.5 83)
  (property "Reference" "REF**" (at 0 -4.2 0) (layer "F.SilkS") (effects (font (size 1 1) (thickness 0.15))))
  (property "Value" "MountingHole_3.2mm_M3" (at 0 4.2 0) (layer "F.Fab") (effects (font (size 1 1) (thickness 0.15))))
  (pad "" np_thru_hole circle (at 0 0) (size 3.2 3.2) (drill 3.2) (layers "*.Cu" "*.Mask")))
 (gr_line (start 99.474874 70.974874) (end 99.474875 83.525126) (stroke (width 0.1) (type default)) (layer "Edge.Cuts"))
 (gr_arc (start 121.5 83.5) (mid 120.474874 85.974874) (end 118 87) (stroke (width 0.1) (type default)) (layer "Edge.Cuts"))
 (gr_arc (start 99.474874 70.974874) (mid 100.5 68.5) (end 102.974874 67.474874) (stroke (width 0.1) (type default)) (layer "Edge.Cuts"))
 (gr_line (start 118 87) (end 102.974874 87.025125) (stroke (width 0.1) (type default)) (layer "Edge.Cuts"))
 (gr_line (start 121.525126 70.974874) (end 121.5 83.5) (stroke (width 0.1) (type default)) (layer "Edge.Cuts"))
 (gr_line (start 102.974874 67.474874) (end 118.025126 67.474874) (stroke (width 0.1) (type default)) (layer "Edge.Cuts"))
 (gr_arc (start 102.974874 87.025125) (mid 100.500001 85.999999) (end 99.474875 83.525126) (stroke (width 0.1) (type default))
  (layer "Edge.Cuts"))
 (gr_arc (start 118.025126 67.474874) (mid 120.5 68.5) (end 121.525126 70.974874) (stroke (width 0.1) (type default)) (layer "Edge.Cuts"))
 (segment (start 117.305 72) (end 117.305 75.995) (width 0.25) (layer "F.Cu") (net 4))
 (segment (start 117.305 75.995) (end 116.3 77) (width 0.25) (layer "F.Cu") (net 4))
 (segment (start 114.7 80.3) (end 113.5 81.5) (width 0.25) (layer "F.Cu") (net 3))
 (segment (start 113.5 83.5) (end 106.5 83.5) (width 0.25) (layer "F.Cu") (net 3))
 (segment (start 114.7 77) (end 114.7 80.3) (width 0.25) (layer "F.Cu") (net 3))
 (segment (start 106.5 83.5) (end 104.5 81.5) (width 0.25) (layer "F.Cu") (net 3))
 (segment (start 113.5 81.5) (end 113.5 83.5) (width 0.25) (layer "F.Cu") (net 3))
 (segment (start 104.5 81.5) (end 104.5 80) (width 0.25) (layer "F.Cu") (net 3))
 (via (at 104.5 80) (size 0.8) (drill 0.4) (layers "F.Cu" "B.Cu") (free yes) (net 3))
 (segment (start 108.695 72) (end 108.695 73.805) (width 0.25) (layer "F.Cu") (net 2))
 (segment (start 106.5 76) (end 106.5 76.975) (width 0.25) (layer "F.Cu") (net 2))
 (segment (start 108.695 73.805) (end 106.5 76) (width 0.25) (layer "F.Cu") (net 2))
 (segment (start 106.5 76.975) (end 105.475 78) (width 0.25) (layer "F.Cu") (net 2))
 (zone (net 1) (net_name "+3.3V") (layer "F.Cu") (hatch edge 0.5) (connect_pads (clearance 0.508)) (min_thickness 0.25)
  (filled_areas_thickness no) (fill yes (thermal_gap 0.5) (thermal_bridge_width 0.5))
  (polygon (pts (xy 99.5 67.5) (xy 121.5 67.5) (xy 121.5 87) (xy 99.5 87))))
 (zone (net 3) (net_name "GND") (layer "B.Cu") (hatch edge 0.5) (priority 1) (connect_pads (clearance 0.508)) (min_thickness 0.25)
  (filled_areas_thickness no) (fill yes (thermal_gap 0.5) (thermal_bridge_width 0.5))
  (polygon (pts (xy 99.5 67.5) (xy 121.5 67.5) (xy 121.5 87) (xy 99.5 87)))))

